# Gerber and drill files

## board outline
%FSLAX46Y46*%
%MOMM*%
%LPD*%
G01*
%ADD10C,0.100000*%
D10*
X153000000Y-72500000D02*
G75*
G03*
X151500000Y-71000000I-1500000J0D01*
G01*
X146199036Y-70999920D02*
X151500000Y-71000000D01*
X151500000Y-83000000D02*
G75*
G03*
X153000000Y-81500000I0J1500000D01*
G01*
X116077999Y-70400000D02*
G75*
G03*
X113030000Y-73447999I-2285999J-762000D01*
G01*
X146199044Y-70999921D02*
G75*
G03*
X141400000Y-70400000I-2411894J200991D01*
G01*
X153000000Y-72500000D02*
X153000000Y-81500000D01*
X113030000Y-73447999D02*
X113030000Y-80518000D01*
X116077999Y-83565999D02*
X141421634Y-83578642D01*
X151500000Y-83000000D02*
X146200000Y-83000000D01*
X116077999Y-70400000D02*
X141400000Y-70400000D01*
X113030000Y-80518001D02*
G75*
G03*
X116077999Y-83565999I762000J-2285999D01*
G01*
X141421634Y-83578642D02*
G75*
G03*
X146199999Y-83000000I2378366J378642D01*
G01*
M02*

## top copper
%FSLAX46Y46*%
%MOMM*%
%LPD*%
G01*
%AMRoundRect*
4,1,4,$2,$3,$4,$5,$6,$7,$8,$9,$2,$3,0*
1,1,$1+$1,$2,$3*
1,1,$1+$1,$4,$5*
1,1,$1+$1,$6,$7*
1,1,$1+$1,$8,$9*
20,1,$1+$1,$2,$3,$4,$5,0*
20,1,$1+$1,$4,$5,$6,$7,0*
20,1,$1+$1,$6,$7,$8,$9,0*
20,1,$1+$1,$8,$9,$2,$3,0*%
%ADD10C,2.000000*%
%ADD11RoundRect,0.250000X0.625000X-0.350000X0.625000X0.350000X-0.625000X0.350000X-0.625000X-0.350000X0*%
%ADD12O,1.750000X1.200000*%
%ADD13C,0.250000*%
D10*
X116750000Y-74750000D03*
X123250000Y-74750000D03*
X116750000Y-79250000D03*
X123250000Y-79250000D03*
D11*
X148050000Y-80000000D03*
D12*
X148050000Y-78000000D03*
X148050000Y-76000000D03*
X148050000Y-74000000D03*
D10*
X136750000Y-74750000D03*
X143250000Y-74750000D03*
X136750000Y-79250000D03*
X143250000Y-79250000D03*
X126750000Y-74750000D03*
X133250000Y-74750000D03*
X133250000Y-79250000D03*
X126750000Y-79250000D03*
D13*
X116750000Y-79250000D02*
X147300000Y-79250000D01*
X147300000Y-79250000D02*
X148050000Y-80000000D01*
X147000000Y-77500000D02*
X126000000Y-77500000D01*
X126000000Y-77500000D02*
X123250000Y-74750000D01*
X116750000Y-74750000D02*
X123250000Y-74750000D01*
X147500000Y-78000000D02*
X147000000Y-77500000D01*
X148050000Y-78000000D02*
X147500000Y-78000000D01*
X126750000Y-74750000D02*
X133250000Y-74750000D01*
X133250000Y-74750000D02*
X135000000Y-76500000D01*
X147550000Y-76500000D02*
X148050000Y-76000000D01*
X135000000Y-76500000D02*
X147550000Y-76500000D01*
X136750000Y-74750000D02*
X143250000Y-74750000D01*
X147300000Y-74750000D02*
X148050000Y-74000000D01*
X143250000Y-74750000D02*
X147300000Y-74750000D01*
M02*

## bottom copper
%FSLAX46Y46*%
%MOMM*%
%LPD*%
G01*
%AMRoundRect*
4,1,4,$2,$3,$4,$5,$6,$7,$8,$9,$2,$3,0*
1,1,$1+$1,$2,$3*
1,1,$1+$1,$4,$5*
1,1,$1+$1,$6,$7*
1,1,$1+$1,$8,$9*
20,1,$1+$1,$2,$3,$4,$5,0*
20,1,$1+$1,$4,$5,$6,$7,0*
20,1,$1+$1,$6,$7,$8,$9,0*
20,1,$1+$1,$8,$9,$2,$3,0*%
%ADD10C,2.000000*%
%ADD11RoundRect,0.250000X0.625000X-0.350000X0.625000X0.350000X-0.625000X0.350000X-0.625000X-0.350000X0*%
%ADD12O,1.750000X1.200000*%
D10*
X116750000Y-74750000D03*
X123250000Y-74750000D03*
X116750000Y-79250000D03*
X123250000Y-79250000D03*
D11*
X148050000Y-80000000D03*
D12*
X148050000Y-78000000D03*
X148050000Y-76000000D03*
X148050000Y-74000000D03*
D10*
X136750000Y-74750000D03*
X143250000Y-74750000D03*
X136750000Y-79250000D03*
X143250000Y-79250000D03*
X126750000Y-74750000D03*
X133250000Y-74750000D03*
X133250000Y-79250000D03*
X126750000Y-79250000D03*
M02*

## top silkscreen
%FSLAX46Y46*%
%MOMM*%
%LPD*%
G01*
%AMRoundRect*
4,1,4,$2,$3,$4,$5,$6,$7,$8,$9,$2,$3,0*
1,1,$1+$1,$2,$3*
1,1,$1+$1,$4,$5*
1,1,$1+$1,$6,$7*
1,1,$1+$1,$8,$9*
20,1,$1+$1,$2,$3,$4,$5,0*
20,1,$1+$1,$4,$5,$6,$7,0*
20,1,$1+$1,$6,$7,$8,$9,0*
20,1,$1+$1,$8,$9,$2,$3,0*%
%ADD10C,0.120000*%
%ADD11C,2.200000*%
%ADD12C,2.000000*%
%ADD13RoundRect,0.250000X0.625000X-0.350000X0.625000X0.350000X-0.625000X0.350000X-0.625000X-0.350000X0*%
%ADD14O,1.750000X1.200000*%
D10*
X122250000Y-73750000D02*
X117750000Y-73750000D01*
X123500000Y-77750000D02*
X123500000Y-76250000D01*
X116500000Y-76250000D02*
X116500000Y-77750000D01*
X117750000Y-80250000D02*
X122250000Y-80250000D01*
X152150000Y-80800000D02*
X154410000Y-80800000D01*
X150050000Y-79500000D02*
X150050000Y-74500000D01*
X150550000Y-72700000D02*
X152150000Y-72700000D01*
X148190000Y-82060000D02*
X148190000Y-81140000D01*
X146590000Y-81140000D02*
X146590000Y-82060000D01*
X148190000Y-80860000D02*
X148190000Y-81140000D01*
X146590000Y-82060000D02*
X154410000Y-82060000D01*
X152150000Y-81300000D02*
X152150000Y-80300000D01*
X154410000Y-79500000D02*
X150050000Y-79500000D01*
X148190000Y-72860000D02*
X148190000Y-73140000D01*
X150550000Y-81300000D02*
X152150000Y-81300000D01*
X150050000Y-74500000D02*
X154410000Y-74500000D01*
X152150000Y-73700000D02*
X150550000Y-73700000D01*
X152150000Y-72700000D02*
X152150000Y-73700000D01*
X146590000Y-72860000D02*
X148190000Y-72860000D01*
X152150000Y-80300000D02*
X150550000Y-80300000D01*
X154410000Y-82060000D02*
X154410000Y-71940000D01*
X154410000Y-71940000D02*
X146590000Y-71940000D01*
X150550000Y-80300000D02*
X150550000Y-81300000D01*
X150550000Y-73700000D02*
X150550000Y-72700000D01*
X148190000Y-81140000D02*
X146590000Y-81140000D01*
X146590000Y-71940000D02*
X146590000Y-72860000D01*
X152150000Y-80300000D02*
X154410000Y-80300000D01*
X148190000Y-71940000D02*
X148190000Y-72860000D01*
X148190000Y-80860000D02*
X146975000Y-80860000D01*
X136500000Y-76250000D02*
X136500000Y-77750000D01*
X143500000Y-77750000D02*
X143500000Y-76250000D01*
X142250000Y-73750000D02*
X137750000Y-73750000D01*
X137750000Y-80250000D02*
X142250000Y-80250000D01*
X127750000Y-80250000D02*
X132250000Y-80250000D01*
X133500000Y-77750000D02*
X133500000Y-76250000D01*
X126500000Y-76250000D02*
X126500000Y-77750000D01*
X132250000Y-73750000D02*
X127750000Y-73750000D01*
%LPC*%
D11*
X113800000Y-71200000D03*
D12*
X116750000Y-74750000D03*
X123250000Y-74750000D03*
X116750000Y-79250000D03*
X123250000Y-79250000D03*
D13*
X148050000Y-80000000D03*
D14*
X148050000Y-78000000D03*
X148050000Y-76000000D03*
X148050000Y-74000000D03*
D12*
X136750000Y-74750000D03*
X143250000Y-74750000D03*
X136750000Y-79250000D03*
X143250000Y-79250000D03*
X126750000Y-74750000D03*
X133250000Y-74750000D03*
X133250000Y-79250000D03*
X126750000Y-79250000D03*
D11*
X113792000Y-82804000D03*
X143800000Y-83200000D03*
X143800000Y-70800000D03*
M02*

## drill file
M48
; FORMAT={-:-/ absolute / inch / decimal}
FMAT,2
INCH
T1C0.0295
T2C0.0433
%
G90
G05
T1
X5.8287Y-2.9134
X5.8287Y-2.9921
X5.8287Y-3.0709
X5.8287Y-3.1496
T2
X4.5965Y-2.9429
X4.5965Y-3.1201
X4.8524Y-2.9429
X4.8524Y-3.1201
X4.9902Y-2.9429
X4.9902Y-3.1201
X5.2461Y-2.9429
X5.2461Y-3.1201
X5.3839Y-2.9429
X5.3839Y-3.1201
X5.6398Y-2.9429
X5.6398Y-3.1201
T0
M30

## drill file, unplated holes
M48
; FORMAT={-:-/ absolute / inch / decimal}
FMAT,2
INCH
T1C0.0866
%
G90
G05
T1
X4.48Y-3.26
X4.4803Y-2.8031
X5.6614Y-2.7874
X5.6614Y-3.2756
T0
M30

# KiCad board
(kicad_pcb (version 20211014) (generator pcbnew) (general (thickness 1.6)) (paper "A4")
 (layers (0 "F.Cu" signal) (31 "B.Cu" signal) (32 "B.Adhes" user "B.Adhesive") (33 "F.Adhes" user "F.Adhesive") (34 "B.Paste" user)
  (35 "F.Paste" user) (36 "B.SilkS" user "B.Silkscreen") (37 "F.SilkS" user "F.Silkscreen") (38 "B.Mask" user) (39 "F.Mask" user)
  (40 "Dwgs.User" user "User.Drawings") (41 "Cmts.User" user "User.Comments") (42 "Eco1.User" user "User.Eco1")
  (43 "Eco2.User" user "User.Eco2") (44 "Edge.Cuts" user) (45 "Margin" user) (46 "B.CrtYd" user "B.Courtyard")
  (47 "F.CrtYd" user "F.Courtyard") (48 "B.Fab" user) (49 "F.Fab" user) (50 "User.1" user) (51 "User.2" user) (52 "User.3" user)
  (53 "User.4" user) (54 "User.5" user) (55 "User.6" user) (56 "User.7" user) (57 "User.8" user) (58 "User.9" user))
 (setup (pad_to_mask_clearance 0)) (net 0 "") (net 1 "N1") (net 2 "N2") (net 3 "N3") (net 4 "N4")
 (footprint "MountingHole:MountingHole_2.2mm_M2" (layer "F.Cu") (at 113.8 71.2)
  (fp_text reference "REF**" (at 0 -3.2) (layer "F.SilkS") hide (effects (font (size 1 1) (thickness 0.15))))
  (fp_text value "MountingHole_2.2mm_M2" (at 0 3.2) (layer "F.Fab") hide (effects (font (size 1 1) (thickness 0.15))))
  (pad "" np_thru_hole circle locked (at 0 0) (size 2.2 2.2) (drill 2.2) (layers F&B.Cu *.Mask)))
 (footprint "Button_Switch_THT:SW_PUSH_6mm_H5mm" (layer "F.Cu") (at 116.75 74.75)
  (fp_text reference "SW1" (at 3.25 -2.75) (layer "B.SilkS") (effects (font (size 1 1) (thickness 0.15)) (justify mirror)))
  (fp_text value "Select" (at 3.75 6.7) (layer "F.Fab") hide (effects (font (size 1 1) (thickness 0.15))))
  (fp_line (start 5.5 -1) (end 1 -1) (layer "F.SilkS") (width 0.12))
  (fp_line (start 6.75 3) (end 6.75 1.5) (layer "F.SilkS") (width 0.12))
  (fp_line (start -0.25 1.5) (end -0.25 3) (layer "F.SilkS") (width 0.12))
  (fp_line (start 1 5.5) (end 5.5 5.5) (layer "F.SilkS") (width 0.12))
  (pad "1" thru_hole circle (at 0 0 90) (size 2 2) (drill 1.1) (layers *.Cu *.Mask) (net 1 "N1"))
  (pad "1" thru_hole circle (at 6.5 0 90) (size 2 2) (drill 1.1) (layers *.Cu *.Mask) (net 1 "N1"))
  (pad "2" thru_hole circle (at 0 4.5 90) (size 2 2) (drill 1.1) (layers *.Cu *.Mask) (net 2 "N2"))
  (pad "2" thru_hole circle (at 6.5 4.5 90) (size 2 2) (drill 1.1) (layers *.Cu *.Mask) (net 2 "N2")))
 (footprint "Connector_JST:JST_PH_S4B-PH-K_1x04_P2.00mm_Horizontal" (layer "F.Cu") (at 148.05 80 90)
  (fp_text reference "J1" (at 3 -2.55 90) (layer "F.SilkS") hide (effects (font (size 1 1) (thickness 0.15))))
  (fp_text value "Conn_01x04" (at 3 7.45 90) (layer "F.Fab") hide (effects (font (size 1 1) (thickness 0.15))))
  (fp_line (start -0.8 4.1) (end -0.8 6.36) (layer "F.SilkS") (width 0.12))
  (fp_line (start 0.5 2) (end 5.5 2) (layer "F.SilkS") (width 0.12))
  (fp_line (start 7.3 2.5) (end 7.3 4.1) (layer "F.SilkS") (width 0.12))
  (fp_line (start -2.06 0.14) (end -1.14 0.14) (layer "F.SilkS") (width 0.12))
  (fp_line (start -1.14 -1.46) (end -2.06 -1.46) (layer "F.SilkS") (width 0.12))
  (fp_line (start -0.86 0.14) (end -1.14 0.14) (layer "F.SilkS") (width 0.12))
  (fp_line (start -2.06 -1.46) (end -2.06 6.36) (layer "F.SilkS") (width 0.12))
  (fp_line (start -1.3 4.1) (end -0.3 4.1) (layer "F.SilkS") (width 0.12))
  (fp_line (start 0.5 6.36) (end 0.5 2) (layer "F.SilkS") (width 0.12))
  (fp_line (start 7.14 0.14) (end 6.86 0.14) (layer "F.SilkS") (width 0.12))
  (fp_line (start -1.3 2.5) (end -1.3 4.1) (layer "F.SilkS") (width 0.12))
  (fp_line (start 5.5 2) (end 5.5 6.36) (layer "F.SilkS") (width 0.12))
  (fp_line (start 6.3 4.1) (end 6.3 2.5) (layer "F.SilkS") (width 0.12))
  (fp_line (start 7.3 4.1) (end 6.3 4.1) (layer "F.SilkS") (width 0.12))
  (fp_line (start 7.14 -1.46) (end 7.14 0.14) (layer "F.SilkS") (width 0.12))
  (fp_line (start -0.3 4.1) (end -0.3 2.5) (layer "F.SilkS") (width 0.12))
  (fp_line (start -2.06 6.36) (end 8.06 6.36) (layer "F.SilkS") (width 0.12))
  (fp_line (start 8.06 6.36) (end 8.06 -1.46) (layer "F.SilkS") (width 0.12))
  (fp_line (start -0.3 2.5) (end -1.3 2.5) (layer "F.SilkS") (width 0.12))
  (fp_line (start 6.3 2.5) (end 7.3 2.5) (layer "F.SilkS") (width 0.12))
  (fp_line (start -1.14 0.14) (end -1.14 -1.46) (layer "F.SilkS") (width 0.12))
  (fp_line (start 8.06 -1.46) (end 7.14 -1.46) (layer "F.SilkS") (width 0.12))
  (fp_line (start -0.3 4.1) (end -0.3 6.36) (layer "F.SilkS") (width 0.12))
  (fp_line (start 8.06 0.14) (end 7.14 0.14) (layer "F.SilkS") (width 0.12))
  (fp_line (start -0.86 0.14) (end -0.86 -1.075) (layer "F.SilkS") (width 0.12))
  (pad "1" thru_hole roundrect (at 0 0 90) (size 1.2 1.75) (drill 0.75) (layers *.Cu *.Mask) (roundrect_rratio 0.2083333333) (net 2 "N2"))
  (pad "2" thru_hole oval (at 2 0 90) (size 1.2 1.75) (drill 0.75) (layers *.Cu *.Mask) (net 1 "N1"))
  (pad "3" thru_hole oval (at 4 0 90) (size 1.2 1.75) (drill 0.75) (layers *.Cu *.Mask) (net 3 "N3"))
  (pad "4" thru_hole oval (at 6 0 90) (size 1.2 1.75) (drill 0.75) (layers *.Cu *.Mask) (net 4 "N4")))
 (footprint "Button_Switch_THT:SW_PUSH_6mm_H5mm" (layer "F.Cu") (at 136.75 74.75)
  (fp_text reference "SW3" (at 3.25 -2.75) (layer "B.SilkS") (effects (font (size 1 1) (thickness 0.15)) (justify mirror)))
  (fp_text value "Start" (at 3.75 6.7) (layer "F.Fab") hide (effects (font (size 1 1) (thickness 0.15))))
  (fp_line (start -0.25 1.5) (end -0.25 3) (layer "F.SilkS") (width 0.12))
  (fp_line (start 6.75 3) (end 6.75 1.5) (layer "F.SilkS") (width 0.12))
  (fp_line (start 5.5 -1) (end 1 -1) (layer "F.SilkS") (width 0.12))
  (fp_line (start 1 5.5) (end 5.5 5.5) (layer "F.SilkS") (width 0.12))
  (pad "1" thru_hole circle (at 0 0 90) (size 2 2) (drill 1.1) (layers *.Cu *.Mask) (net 4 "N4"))
  (pad "1" thru_hole circle (at 6.5 0 90) (size 2 2) (drill 1.1) (layers *.Cu *.Mask) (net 4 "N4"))
  (pad "2" thru_hole circle (at 0 4.5 90) (size 2 2) (drill 1.1) (layers *.Cu *.Mask) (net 2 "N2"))
  (pad "2" thru_hole circle (at 6.5 4.5 90) (size 2 2) (drill 1.1) (layers *.Cu *.Mask) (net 2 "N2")))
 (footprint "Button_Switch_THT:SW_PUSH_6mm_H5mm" (layer "F.Cu") (at 126.75 74.75)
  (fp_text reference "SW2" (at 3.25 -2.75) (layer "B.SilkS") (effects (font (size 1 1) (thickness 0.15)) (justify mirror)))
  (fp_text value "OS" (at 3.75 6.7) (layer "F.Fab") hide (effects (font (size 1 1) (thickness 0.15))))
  (fp_line (start 1 5.5) (end 5.5 5.5) (layer "F.SilkS") (width 0.12))
  (fp_line (start 6.75 3) (end 6.75 1.5) (layer "F.SilkS") (width 0.12))
  (fp_line (start -0.25 1.5) (end -0.25 3) (layer "F.SilkS") (width 0.12))
  (fp_line (start 5.5 -1) (end 1 -1) (layer "F.SilkS") (width 0.12))
  (pad "1" thru_hole circle (at 0 0 90) (size 2 2) (drill 1.1) (layers *.Cu *.Mask) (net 3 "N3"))
  (pad "1" thru_hole circle (at 6.5 0 90) (size 2 2) (drill 1.1) (layers *.Cu *.Mask) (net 3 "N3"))
  (pad "2" thru_hole circle (at 6.5 4.5 90) (size 2 2) (drill 1.1) (layers *.Cu *.Mask) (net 2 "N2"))
  (pad "2" thru_hole circle (at 0 4.5 90) (size 2 2) (drill 1.1) (layers *.Cu *.Mask) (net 2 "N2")))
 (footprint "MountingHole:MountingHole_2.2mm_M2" (layer "F.Cu") (at 113.792 82.804)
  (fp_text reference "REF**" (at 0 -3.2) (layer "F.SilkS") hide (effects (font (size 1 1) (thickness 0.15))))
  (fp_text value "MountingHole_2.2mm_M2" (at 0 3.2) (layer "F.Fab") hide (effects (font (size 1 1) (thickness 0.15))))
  (pad "" np_thru_hole circle locked (at 0 0) (size 2.2 2.2) (drill 2.2) (layers *.Cu *.Mask)))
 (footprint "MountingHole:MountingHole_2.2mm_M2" (layer "F.Cu") (at 143.8 83.2)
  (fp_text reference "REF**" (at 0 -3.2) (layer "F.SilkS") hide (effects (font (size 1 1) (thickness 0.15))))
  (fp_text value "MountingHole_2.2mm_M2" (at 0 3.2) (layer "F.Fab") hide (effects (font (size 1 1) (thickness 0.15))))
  (pad "" np_thru_hole circle locked (at 0 0) (size 2.2 2.2) (drill 2.2) (layers F&B.Cu *.Mask)))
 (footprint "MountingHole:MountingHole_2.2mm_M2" (layer "F.Cu") (at 143.8 70.8)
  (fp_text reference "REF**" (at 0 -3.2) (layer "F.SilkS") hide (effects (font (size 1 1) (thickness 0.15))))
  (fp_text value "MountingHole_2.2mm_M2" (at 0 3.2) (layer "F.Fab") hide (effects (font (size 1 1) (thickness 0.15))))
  (pad "" np_thru_hole circle locked (at 0 0) (size 2.2 2.2) (drill 2.2) (layers F&B.Cu *.Mask)))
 (gr_arc (start 151.5 71) (mid 152.56066 71.43934) (end 153 72.5) (layer "Edge.Cuts") (width 0.1))
 (gr_line (start 146.199036 70.99992) (end 151.5 71) (layer "Edge.Cuts") (width 0.1))
 (gr_arc (start 153 81.5) (mid 152.56066 82.56066) (end 151.5 83) (layer "Edge.Cuts") (width 0.1))
 (gr_arc (start 113.03 73.447999) (mid 112.088117 69.458117) (end 116.077999 70.4) (layer "Edge.Cuts") (width 0.1))
 (gr_arc (start 141.4 70.4) (mid 144.087361 68.39737) (end 146.199036 70.99992) (layer "Edge.Cuts") (width 0.1))
 (gr_line (start 153 72.5) (end 153 81.5) (layer "Edge.Cuts") (width 0.1))
 (gr_line (start 113.03 73.447999) (end 113.03 80.518) (layer "Edge.Cuts") (width 0.1))
 (gr_line (start 116.077999 83.565999) (end 141.421634 83.578642) (layer "Edge.Cuts") (width 0.1))
 (gr_line (start 151.5 83) (end 146.2 83) (layer "Edge.Cuts") (width 0.1))
 (gr_line (start 116.077999 70.4) (end 141.4 70.4) (layer "Edge.Cuts") (width 0.1))
 (gr_arc (start 116.077999 83.565999) (mid 112.088117 84.507882) (end 113.03 80.518) (layer "Edge.Cuts") (width 0.1))
 (gr_arc (start 146.199999 83) (mid 144.089523 85.590852) (end 141.421634 83.578642) (layer "Edge.Cuts") (width 0.1))
 (segment (start 116.75 79.25) (end 147.3 79.25) (width 0.25) (layer "F.Cu") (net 2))
 (segment (start 147.3 79.25) (end 148.05 80) (width 0.25) (layer "F.Cu") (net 2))
 (segment (start 147 77.5) (end 126 77.5) (width 0.25) (layer "F.Cu") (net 1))
 (segment (start 126 77.5) (end 123.25 74.75) (width 0.25) (layer "F.Cu") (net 1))
 (segment (start 116.75 74.75) (end 123.25 74.75) (width 0.25) (layer "F.Cu") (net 1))
 (segment (start 147.5 78) (end 147 77.5) (width 0.25) (layer "F.Cu") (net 1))
 (segment (start 148.05 78) (end 147.5 78) (width 0.25) (layer "F.Cu") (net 1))
 (segment (start 126.75 74.75) (end 133.25 74.75) (width 0.25) (layer "F.Cu") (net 3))
 (segment (start 133.25 74.75) (end 135 76.5) (width 0.25) (layer "F.Cu") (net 3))
 (segment (start 147.55 76.5) (end 148.05 76) (width 0.25) (layer "F.Cu") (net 3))
 (segment (start 135 76.5) (end 147.55 76.5) (width 0.25) (layer "F.Cu") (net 3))
 (segment (start 136.75 74.75) (end 143.25 74.75) (width 0.25) (layer "F.Cu") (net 4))
 (segment (start 147.3 74.75) (end 148.05 74) (width 0.25) (layer "F.Cu") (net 4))
 (segment (start 143.25 74.75) (end 147.3 74.75) (width 0.25) (layer "F.Cu") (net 4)))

